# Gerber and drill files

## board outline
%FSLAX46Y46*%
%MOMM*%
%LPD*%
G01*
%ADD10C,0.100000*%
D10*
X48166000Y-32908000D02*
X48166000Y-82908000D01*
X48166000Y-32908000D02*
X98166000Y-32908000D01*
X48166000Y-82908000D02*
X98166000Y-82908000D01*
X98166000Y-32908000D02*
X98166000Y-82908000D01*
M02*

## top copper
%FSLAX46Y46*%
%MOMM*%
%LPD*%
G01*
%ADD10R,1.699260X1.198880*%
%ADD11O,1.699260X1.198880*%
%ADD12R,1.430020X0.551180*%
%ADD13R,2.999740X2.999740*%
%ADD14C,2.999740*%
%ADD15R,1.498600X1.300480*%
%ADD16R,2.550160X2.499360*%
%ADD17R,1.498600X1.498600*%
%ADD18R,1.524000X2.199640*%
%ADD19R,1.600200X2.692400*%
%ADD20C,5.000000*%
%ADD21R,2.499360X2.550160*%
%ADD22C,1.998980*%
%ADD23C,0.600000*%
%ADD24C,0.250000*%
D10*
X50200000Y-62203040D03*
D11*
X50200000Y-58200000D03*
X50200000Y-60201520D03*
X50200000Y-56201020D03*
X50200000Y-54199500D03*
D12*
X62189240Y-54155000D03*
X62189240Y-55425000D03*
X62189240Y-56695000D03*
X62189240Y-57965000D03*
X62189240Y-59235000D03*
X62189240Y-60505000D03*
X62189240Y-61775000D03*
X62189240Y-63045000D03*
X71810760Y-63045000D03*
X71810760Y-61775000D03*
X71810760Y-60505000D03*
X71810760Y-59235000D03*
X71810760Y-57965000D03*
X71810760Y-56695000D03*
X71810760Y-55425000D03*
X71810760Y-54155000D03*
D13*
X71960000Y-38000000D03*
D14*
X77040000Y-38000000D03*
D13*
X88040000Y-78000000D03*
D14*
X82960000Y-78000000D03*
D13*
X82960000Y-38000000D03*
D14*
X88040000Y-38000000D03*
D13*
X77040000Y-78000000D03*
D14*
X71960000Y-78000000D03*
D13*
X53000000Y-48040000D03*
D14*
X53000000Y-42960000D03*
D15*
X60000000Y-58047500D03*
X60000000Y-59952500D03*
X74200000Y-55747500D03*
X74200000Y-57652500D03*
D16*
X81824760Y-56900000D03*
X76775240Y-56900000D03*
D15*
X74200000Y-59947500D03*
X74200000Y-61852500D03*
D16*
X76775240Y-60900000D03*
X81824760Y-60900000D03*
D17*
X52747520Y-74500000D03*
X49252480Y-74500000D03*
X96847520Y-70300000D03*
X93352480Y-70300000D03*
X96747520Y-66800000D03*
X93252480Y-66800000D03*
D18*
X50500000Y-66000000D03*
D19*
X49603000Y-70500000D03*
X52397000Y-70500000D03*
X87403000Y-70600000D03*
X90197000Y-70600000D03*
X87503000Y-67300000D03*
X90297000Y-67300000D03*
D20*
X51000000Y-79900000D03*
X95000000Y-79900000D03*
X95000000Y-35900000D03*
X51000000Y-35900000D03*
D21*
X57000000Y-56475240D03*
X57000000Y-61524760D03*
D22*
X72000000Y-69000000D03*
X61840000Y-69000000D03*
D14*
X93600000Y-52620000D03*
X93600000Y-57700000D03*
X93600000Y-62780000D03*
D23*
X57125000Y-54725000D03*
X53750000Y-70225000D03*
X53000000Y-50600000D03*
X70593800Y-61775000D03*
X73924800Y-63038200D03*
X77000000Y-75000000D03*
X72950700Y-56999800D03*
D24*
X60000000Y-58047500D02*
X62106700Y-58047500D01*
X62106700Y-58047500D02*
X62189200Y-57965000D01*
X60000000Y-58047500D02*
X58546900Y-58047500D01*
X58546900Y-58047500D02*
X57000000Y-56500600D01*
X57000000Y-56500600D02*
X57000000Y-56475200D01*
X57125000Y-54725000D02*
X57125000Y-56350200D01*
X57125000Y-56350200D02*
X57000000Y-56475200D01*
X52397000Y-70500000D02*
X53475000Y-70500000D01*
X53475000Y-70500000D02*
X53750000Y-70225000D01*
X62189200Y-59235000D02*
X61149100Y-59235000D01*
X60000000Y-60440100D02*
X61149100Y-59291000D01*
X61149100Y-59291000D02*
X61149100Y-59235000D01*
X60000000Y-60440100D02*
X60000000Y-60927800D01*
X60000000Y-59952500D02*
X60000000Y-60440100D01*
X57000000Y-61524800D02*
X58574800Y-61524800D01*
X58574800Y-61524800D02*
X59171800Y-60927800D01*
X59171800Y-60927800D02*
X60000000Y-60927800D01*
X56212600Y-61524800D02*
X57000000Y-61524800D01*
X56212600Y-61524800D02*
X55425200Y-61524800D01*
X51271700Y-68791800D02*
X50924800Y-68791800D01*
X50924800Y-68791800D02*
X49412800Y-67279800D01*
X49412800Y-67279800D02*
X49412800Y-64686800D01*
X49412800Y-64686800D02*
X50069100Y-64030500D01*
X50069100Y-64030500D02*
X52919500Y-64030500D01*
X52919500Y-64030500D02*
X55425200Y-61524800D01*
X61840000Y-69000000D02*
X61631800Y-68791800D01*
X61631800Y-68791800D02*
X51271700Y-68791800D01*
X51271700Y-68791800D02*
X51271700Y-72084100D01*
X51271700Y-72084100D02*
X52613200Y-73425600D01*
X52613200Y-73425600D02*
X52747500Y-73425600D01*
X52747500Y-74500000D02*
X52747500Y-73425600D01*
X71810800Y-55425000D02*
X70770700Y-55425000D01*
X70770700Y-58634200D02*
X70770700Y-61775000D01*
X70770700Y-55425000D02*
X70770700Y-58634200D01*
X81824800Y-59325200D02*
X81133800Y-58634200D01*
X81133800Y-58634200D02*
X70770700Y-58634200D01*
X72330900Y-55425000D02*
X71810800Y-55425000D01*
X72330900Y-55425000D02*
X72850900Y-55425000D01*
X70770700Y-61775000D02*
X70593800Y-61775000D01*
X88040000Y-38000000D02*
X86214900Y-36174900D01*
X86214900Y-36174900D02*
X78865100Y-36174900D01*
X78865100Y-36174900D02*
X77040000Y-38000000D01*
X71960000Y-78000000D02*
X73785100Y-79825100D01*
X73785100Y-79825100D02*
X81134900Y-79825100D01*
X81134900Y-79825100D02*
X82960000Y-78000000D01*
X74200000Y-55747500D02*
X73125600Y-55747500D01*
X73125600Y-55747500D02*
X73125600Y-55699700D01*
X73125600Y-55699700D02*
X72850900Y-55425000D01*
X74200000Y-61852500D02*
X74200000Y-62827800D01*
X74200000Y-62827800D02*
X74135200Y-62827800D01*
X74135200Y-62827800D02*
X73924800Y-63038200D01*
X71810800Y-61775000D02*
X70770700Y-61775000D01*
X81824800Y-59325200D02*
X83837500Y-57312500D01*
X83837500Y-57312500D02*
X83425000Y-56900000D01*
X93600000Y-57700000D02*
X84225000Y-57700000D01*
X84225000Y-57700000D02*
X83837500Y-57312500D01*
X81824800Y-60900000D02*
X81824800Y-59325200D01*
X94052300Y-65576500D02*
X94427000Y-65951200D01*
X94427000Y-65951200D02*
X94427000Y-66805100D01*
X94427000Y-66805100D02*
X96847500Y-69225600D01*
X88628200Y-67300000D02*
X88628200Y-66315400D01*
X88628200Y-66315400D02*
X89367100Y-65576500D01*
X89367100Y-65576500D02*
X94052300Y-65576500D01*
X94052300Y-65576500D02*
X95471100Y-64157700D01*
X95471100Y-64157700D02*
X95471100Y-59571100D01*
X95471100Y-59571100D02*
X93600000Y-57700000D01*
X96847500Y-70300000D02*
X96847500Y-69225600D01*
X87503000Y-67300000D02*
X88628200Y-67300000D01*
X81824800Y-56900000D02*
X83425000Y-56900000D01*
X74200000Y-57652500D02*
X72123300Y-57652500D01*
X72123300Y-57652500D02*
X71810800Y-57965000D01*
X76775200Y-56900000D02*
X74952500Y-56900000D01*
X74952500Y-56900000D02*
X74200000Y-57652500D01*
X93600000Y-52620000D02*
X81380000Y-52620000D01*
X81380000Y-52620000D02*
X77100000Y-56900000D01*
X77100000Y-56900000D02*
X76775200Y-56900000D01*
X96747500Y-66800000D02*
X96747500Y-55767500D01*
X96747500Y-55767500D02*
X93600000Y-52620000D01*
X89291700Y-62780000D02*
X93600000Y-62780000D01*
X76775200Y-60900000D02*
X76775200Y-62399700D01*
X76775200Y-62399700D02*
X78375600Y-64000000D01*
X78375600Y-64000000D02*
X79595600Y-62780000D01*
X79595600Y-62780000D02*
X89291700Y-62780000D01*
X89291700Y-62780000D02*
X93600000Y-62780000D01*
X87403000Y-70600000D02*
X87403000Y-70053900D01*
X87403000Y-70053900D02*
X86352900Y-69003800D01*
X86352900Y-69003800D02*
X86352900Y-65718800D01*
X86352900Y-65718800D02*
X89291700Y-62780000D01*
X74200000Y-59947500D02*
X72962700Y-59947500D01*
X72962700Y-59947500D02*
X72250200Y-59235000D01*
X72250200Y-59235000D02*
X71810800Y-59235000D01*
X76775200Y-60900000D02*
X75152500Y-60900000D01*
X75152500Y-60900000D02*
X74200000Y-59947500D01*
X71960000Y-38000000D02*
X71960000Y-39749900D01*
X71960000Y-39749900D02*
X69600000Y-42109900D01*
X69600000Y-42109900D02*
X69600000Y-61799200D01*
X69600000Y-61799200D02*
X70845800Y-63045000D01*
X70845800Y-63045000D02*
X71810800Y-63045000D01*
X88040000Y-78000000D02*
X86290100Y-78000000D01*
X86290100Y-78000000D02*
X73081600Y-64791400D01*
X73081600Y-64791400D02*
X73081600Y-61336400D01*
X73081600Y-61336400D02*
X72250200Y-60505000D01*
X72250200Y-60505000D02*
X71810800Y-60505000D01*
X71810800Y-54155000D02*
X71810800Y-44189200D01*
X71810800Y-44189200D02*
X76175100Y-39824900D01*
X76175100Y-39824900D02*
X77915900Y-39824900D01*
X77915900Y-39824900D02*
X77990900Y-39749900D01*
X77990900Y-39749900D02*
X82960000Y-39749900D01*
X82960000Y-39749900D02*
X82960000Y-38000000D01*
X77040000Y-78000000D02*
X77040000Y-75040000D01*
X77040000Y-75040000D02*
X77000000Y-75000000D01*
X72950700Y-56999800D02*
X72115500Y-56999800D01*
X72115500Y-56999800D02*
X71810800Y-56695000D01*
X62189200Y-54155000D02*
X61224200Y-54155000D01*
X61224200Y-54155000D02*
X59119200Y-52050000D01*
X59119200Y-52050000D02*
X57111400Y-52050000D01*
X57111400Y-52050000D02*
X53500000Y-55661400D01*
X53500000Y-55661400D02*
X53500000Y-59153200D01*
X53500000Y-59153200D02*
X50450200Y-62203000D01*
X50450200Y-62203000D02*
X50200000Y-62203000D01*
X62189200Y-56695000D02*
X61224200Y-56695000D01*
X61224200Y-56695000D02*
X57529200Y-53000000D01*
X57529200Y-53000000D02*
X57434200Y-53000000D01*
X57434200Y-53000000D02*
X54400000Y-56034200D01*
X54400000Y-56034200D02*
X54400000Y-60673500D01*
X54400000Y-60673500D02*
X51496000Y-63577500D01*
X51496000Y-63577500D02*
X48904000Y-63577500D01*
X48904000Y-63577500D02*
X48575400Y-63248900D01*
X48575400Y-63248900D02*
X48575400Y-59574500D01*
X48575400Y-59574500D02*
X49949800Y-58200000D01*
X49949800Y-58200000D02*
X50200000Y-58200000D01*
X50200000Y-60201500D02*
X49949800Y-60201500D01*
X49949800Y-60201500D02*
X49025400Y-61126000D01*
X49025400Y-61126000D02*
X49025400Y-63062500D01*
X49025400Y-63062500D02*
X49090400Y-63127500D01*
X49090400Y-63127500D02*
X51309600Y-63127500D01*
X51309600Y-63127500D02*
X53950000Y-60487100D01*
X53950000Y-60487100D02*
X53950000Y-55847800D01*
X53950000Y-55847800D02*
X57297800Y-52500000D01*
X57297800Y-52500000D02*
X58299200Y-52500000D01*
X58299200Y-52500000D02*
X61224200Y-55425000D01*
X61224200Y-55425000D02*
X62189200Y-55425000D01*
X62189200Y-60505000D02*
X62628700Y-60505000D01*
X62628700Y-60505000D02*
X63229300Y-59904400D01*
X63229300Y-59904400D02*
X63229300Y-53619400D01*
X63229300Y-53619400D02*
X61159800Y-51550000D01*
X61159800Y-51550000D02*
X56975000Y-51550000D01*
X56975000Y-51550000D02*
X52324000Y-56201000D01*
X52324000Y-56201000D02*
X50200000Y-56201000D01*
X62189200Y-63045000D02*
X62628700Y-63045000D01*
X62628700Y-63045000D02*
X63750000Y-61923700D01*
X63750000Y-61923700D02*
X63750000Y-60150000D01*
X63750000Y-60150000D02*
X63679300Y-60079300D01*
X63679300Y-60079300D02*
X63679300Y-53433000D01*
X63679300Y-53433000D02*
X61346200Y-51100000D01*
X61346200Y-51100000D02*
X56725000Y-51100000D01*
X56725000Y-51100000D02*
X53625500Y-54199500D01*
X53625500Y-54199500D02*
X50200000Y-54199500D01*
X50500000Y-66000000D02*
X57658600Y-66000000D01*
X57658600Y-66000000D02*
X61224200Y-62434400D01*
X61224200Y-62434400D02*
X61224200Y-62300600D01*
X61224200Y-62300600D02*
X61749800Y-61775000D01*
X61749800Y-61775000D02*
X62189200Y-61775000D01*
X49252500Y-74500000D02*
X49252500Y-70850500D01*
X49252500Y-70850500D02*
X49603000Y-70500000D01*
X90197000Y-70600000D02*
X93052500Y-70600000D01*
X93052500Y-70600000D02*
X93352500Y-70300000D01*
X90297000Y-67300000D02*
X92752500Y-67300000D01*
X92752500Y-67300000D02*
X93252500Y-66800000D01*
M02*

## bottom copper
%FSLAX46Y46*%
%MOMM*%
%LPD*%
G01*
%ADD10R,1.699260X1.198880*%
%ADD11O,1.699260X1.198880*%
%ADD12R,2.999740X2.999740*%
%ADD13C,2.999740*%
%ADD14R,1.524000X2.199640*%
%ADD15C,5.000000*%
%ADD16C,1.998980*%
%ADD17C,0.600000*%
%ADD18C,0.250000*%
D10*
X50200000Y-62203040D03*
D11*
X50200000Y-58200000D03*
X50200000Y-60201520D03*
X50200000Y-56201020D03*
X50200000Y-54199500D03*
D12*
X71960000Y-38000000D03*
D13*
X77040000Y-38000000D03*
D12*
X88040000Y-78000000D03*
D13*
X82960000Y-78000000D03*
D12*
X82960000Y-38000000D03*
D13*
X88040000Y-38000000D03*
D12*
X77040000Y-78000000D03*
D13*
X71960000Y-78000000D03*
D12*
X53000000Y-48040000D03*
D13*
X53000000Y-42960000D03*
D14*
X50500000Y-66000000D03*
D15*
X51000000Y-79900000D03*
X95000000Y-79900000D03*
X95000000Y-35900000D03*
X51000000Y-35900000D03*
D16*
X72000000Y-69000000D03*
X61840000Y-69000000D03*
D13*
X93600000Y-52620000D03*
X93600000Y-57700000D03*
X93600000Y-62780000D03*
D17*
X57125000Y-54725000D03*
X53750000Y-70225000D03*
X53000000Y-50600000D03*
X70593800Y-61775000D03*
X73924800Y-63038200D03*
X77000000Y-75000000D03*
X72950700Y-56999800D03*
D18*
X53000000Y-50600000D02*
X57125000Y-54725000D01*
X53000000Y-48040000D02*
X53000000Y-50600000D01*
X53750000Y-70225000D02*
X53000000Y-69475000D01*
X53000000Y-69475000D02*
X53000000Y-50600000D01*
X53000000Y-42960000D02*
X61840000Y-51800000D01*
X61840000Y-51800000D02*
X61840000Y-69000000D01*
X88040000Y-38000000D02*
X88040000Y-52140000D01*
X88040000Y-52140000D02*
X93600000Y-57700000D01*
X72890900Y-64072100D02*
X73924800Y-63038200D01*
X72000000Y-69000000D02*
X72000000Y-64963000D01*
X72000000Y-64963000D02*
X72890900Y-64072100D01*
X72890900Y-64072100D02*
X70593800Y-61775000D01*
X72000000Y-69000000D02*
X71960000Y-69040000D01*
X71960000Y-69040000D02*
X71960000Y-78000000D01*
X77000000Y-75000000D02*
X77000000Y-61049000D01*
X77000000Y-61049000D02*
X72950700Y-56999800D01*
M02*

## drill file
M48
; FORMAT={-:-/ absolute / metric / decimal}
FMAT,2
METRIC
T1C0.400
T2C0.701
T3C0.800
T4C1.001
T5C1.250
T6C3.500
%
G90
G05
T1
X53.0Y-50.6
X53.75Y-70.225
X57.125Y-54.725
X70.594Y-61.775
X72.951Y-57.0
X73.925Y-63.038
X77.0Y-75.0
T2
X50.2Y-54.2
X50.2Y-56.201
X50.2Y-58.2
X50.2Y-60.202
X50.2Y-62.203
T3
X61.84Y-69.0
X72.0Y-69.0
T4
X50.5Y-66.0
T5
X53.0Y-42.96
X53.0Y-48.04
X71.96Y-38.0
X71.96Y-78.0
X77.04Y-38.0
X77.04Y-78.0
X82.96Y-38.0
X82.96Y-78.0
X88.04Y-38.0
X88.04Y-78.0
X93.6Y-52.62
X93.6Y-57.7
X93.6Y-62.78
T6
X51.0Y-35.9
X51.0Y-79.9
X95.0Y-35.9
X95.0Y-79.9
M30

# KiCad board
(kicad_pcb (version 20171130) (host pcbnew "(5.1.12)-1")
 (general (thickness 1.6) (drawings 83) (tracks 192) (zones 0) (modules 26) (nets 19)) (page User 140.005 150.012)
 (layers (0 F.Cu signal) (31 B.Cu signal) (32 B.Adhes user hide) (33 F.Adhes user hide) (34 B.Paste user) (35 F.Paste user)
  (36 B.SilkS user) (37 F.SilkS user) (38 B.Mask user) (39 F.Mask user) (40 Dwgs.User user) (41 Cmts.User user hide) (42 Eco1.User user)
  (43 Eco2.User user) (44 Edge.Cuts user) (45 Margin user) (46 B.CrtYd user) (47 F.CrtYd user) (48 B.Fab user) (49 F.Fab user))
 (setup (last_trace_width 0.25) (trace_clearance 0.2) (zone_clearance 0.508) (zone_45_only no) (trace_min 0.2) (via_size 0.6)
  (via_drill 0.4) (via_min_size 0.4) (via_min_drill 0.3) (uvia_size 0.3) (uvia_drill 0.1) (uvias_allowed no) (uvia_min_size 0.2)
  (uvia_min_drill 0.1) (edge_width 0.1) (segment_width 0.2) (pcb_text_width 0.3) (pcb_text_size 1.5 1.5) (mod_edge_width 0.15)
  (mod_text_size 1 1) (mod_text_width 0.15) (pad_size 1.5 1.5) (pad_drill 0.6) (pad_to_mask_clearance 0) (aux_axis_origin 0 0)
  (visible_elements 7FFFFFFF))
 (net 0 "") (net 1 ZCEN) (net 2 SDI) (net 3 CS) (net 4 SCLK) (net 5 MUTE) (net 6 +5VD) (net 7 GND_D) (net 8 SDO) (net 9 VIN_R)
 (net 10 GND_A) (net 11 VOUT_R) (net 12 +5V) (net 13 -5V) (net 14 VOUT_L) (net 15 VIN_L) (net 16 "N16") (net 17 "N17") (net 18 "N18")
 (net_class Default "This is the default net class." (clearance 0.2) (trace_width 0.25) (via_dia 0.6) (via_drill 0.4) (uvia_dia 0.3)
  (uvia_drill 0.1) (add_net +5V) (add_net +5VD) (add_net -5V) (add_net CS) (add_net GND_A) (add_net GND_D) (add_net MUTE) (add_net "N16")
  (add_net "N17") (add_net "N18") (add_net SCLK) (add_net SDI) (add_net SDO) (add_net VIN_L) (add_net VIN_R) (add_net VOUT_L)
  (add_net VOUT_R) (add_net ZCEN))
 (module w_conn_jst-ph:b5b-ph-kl (layer F.Cu) (at 50.2 58.2 90)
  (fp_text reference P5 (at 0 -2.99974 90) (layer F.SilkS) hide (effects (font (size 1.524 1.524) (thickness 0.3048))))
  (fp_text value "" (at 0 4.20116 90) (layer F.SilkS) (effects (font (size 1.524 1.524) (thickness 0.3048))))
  (pad 1 thru_hole rect (at -4.00304 0 90) (size 1.19888 1.69926) (drill 0.70104) (layers *.Cu *.Mask F.SilkS) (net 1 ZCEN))
  (pad 3 thru_hole oval (at 0 0 90) (size 1.19888 1.69926) (drill 0.70104) (layers *.Cu *.Mask F.SilkS) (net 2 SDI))
  (pad 2 thru_hole oval (at -2.00152 0 90) (size 1.19888 1.69926) (drill 0.70104) (layers *.Cu *.Mask F.SilkS) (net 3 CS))
  (pad 4 thru_hole oval (at 1.99898 0 90) (size 1.19888 1.69926) (drill 0.70104) (layers *.Cu *.Mask F.SilkS) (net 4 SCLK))
  (pad 5 thru_hole oval (at 4.0005 0 90) (size 1.19888 1.69926) (drill 0.70104) (layers *.Cu *.Mask F.SilkS) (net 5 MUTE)))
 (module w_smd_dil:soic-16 (layer F.Cu) (at 67 58.6 270)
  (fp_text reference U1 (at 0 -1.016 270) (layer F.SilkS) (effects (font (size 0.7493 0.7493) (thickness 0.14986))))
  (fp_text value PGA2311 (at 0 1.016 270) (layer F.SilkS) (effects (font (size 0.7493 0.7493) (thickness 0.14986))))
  (pad 1 smd rect (at -4.445 4.81076 270) (size 0.55118 1.43002) (layers F.Cu F.Paste F.Mask) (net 1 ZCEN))
  (pad 2 smd rect (at -3.175 4.81076 270) (size 0.55118 1.43002) (layers F.Cu F.Paste F.Mask) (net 3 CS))
  (pad 3 smd rect (at -1.905 4.81076 270) (size 0.55118 1.43002) (layers F.Cu F.Paste F.Mask) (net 2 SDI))
  (pad 4 smd rect (at -0.635 4.81076 270) (size 0.55118 1.43002) (layers F.Cu F.Paste F.Mask) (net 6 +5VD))
  (pad 5 smd rect (at 0.635 4.81076 270) (size 0.55118 1.43002) (layers F.Cu F.Paste F.Mask) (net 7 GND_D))
  (pad 6 smd rect (at 1.905 4.81076 270) (size 0.55118 1.43002) (layers F.Cu F.Paste F.Mask) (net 4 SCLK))
  (pad 7 smd rect (at 3.175 4.81076 270) (size 0.55118 1.43002) (layers F.Cu F.Paste F.Mask) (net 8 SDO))
  (pad 8 smd rect (at 4.445 4.81076 270) (size 0.55118 1.43002) (layers F.Cu F.Paste F.Mask) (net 5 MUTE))
  (pad 9 smd rect (at 4.445 -4.81076 270) (size 0.55118 1.43002) (layers F.Cu F.Paste F.Mask) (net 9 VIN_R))
  (pad 10 smd rect (at 3.175 -4.81076 270) (size 0.55118 1.43002) (layers F.Cu F.Paste F.Mask) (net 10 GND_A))
  (pad 11 smd rect (at 1.905 -4.81076 270) (size 0.55118 1.43002) (layers F.Cu F.Paste F.Mask) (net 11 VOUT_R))
  (pad 12 smd rect (at 0.635 -4.81076 270) (size 0.55118 1.43002) (layers F.Cu F.Paste F.Mask) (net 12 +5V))
  (pad 13 smd rect (at -0.635 -4.81076 270) (size 0.55118 1.43002) (layers F.Cu F.Paste F.Mask) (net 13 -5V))
  (pad 14 smd rect (at -1.905 -4.81076 270) (size 0.55118 1.43002) (layers F.Cu F.Paste F.Mask) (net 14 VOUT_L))
  (pad 15 smd rect (at -3.175 -4.81076 270) (size 0.55118 1.43002) (layers F.Cu F.Paste F.Mask) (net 10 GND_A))
  (pad 16 smd rect (at -4.445 -4.81076 270) (size 0.55118 1.43002) (layers F.Cu F.Paste F.Mask) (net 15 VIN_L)))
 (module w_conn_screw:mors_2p (layer F.Cu) (at 74.5 38)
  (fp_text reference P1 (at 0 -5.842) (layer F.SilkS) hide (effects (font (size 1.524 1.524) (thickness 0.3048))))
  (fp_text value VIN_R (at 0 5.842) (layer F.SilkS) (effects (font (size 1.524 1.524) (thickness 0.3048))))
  (pad 1 thru_hole rect (at -2.54 0) (size 2.99974 2.99974) (drill 1.24968) (layers *.Cu *.Mask F.SilkS) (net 9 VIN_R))
  (pad 2 thru_hole circle (at 2.54 0) (size 2.99974 2.99974) (drill 1.24968) (layers *.Cu *.Mask F.SilkS) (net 10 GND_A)))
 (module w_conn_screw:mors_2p (layer F.Cu) (at 85.5 78 180)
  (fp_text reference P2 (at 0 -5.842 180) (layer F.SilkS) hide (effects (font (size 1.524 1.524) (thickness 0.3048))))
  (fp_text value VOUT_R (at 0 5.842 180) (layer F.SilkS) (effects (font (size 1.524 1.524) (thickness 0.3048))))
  (pad 1 thru_hole rect (at -2.54 0 180) (size 2.99974 2.99974) (drill 1.24968) (layers *.Cu *.Mask F.SilkS) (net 11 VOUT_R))
  (pad 2 thru_hole circle (at 2.54 0 180) (size 2.99974 2.99974) (drill 1.24968) (layers *.Cu *.Mask F.SilkS) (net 10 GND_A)))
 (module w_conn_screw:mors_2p (layer F.Cu) (at 85.5 38)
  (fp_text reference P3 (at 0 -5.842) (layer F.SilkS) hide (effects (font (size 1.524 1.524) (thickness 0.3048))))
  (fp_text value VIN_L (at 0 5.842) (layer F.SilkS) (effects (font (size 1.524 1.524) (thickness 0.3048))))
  (pad 1 thru_hole rect (at -2.54 0) (size 2.99974 2.99974) (drill 1.24968) (layers *.Cu *.Mask F.SilkS) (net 15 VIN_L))
  (pad 2 thru_hole circle (at 2.54 0) (size 2.99974 2.99974) (drill 1.24968) (layers *.Cu *.Mask F.SilkS) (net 10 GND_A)))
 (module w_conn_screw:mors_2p (layer F.Cu) (at 74.5 78 180)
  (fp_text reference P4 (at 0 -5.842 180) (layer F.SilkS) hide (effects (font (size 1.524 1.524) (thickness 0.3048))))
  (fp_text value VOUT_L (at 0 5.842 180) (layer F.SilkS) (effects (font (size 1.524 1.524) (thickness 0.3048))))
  (pad 1 thru_hole rect (at -2.54 0 180) (size 2.99974 2.99974) (drill 1.24968) (layers *.Cu *.Mask F.SilkS) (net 14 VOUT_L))
  (pad 2 thru_hole circle (at 2.54 0 180) (size 2.99974 2.99974) (drill 1.24968) (layers *.Cu *.Mask F.SilkS) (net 10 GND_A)))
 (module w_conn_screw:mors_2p (layer F.Cu) (at 53 45.5 90)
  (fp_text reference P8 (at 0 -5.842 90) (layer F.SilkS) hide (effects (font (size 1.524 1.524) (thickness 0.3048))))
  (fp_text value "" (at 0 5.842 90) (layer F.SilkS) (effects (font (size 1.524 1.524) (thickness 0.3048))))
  (pad 1 thru_hole rect (at -2.54 0 90) (size 2.99974 2.99974) (drill 1.24968) (layers *.Cu *.Mask F.SilkS) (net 6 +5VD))
  (pad 2 thru_hole circle (at 2.54 0 90) (size 2.99974 2.99974) (drill 1.24968) (layers *.Cu *.Mask F.SilkS) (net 7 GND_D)))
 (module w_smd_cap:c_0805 (layer F.Cu) (at 60 59 90)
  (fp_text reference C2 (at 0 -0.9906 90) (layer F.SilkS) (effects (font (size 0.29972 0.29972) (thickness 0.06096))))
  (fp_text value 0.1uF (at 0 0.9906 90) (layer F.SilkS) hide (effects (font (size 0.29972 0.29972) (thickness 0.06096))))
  (pad 1 smd rect (at 0.9525 0 90) (size 1.30048 1.4986) (layers F.Cu F.Paste F.Mask) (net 6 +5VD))
  (pad 2 smd rect (at -0.9525 0 90) (size 1.30048 1.4986) (layers F.Cu F.Paste F.Mask) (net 7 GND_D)))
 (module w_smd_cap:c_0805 (layer F.Cu) (at 74.2 56.7 90)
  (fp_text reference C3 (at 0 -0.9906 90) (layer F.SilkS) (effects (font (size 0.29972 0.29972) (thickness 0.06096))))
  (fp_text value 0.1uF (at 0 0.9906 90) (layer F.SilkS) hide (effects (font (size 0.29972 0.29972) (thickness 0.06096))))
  (pad 1 smd rect (at 0.9525 0 90) (size 1.30048 1.4986) (layers F.Cu F.Paste F.Mask) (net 10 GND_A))
  (pad 2 smd rect (at -0.9525 0 90) (size 1.30048 1.4986) (layers F.Cu F.Paste F.Mask) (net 13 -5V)))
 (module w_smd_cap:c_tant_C (layer F.Cu) (at 79.3 56.9)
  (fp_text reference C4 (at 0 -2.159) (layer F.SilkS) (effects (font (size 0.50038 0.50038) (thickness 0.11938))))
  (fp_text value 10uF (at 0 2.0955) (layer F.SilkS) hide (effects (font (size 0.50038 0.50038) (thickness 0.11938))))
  (pad 1 smd rect (at 2.52476 0) (size 2.55016 2.49936) (layers F.Cu F.Paste F.Mask) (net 10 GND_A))
  (pad 2 smd rect (at -2.52476 0) (size 2.55016 2.49936) (layers F.Cu F.Paste F.Mask) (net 13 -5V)))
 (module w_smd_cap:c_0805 (layer F.Cu) (at 74.2 60.9 90)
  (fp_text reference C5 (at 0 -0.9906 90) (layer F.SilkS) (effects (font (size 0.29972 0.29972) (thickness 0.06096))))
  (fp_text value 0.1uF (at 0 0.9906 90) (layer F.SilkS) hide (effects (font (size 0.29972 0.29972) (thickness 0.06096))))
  (pad 1 smd rect (at 0.9525 0 90) (size 1.30048 1.4986) (layers F.Cu F.Paste F.Mask) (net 12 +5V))
  (pad 2 smd rect (at -0.9525 0 90) (size 1.30048 1.4986) (layers F.Cu F.Paste F.Mask) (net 10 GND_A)))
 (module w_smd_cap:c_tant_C (layer F.Cu) (at 79.3 60.9 180)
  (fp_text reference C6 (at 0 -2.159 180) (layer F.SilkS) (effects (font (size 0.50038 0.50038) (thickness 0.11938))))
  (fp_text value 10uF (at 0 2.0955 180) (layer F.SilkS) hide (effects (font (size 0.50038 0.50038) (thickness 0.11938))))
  (pad 1 smd rect (at 2.52476 0 180) (size 2.55016 2.49936) (layers F.Cu F.Paste F.Mask) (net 12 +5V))
  (pad 2 smd rect (at -2.52476 0 180) (size 2.55016 2.49936) (layers F.Cu F.Paste F.Mask) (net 10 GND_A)))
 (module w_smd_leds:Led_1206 (layer F.Cu) (at 51 74.5 180)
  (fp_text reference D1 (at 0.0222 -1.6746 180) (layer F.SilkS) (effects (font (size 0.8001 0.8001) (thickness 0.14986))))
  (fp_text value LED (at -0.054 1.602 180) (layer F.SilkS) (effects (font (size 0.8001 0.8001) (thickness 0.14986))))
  (pad 1 smd rect (at -1.74752 0 180) (size 1.4986 1.4986) (layers F.Cu F.Paste F.Mask) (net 7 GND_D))
  (pad 2 smd rect (at 1.74752 0 180) (size 1.4986 1.4986) (layers F.Cu F.Paste F.Mask) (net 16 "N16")))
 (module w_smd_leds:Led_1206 (layer F.Cu) (at 95.1 70.3 180)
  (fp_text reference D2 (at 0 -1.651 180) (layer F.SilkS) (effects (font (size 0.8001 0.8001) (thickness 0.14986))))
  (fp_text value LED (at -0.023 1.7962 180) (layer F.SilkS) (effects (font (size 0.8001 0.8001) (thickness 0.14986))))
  (pad 1 smd rect (at -1.74752 0 180) (size 1.4986 1.4986) (layers F.Cu F.Paste F.Mask) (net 10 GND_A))
  (pad 2 smd rect (at 1.74752 0 180) (size 1.4986 1.4986) (layers F.Cu F.Paste F.Mask) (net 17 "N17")))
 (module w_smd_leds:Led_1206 (layer F.Cu) (at 95 66.8 180)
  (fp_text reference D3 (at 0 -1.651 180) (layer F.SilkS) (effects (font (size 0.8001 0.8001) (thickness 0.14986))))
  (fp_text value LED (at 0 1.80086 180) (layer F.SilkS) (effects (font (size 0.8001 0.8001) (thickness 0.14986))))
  (pad 1 smd rect (at -1.74752 0 180) (size 1.4986 1.4986) (layers F.Cu F.Paste F.Mask) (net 13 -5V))
  (pad 2 smd rect (at 1.74752 0 180) (size 1.4986 1.4986) (layers F.Cu F.Paste F.Mask) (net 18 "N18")))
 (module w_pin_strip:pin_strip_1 (layer F.Cu) (at 50.5 66)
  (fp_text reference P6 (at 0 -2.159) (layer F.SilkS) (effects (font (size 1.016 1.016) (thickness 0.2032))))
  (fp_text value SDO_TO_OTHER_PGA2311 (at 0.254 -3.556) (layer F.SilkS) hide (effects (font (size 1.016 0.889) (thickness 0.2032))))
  (pad 1 thru_hole rect (at 0 0) (size 1.524 2.19964) (drill 1.00076) (layers *.Cu *.Mask F.SilkS) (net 8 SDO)))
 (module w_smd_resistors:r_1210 (layer F.Cu) (at 51 70.5 180)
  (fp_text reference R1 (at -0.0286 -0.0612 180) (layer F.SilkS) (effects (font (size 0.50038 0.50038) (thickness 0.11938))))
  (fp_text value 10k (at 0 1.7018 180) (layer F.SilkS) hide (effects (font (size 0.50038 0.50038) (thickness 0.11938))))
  (pad 1 smd rect (at 1.397 0 180) (size 1.6002 2.6924) (layers F.Cu F.Paste F.Mask) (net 16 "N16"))
  (pad 2 smd rect (at -1.397 0 180) (size 1.6002 2.6924) (layers F.Cu F.Paste F.Mask) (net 6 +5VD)))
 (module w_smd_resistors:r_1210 (layer F.Cu) (at 88.8 70.6 180)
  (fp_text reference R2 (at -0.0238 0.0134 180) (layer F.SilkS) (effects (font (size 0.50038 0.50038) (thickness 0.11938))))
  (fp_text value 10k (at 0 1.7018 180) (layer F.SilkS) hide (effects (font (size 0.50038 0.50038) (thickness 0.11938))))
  (pad 1 smd rect (at 1.397 0 180) (size 1.6002 2.6924) (layers F.Cu F.Paste F.Mask) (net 12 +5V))
  (pad 2 smd rect (at -1.397 0 180) (size 1.6002 2.6924) (layers F.Cu F.Paste F.Mask) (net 17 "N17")))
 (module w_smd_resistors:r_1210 (layer F.Cu) (at 88.9 67.3 180)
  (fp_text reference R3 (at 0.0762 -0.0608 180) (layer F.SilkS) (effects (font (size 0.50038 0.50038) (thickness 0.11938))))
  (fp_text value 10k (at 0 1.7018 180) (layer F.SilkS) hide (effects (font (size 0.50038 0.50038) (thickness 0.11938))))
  (pad 1 smd rect (at 1.397 0 180) (size 1.6002 2.6924) (layers F.Cu F.Paste F.Mask) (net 10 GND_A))
  (pad 2 smd rect (at -1.397 0 180) (size 1.6002 2.6924) (layers F.Cu F.Paste F.Mask) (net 18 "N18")))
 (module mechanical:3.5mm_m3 (layer F.Cu) (at 51 80)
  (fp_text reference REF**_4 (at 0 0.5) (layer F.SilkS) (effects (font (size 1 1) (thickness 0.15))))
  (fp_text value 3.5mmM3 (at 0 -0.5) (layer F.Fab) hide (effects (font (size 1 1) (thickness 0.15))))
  (pad 1 thru_hole circle (at 0 -0.1) (size 5 5) (drill 3.5) (layers *.Cu *.Mask F.SilkS)))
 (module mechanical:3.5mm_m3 (layer F.Cu) (at 95 80)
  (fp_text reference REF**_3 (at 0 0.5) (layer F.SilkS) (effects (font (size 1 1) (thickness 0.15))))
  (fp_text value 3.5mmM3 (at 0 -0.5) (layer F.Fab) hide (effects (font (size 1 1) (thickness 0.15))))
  (pad 1 thru_hole circle (at 0 -0.1) (size 5 5) (drill 3.5) (layers *.Cu *.Mask F.SilkS)))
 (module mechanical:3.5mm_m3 (layer F.Cu) (at 95 36)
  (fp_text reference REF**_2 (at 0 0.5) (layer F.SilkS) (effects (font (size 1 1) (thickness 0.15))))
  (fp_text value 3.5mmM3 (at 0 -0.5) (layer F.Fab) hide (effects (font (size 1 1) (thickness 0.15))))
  (pad 1 thru_hole circle (at 0 -0.1) (size 5 5) (drill 3.5) (layers *.Cu *.Mask F.SilkS)))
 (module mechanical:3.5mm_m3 (layer F.Cu) (at 51 36)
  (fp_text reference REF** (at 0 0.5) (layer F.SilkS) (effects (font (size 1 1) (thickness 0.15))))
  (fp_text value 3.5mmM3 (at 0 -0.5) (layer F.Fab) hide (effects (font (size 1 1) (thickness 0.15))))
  (pad 1 thru_hole circle (at 0 -0.1) (size 5 5) (drill 3.5) (layers *.Cu *.Mask F.SilkS)))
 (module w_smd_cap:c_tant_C (layer F.Cu) (at 57 59 90)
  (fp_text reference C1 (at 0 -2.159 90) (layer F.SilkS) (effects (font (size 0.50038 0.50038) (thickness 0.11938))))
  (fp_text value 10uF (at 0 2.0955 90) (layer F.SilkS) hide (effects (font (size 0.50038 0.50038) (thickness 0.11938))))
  (pad 1 smd rect (at 2.52476 0 90) (size 2.55016 2.49936) (layers F.Cu F.Paste F.Mask) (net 6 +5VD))
  (pad 2 smd rect (at -2.52476 0 90) (size 2.55016 2.49936) (layers F.Cu F.Paste F.Mask) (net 7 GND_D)))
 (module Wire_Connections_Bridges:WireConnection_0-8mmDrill (layer F.Cu) (at 72 69 180)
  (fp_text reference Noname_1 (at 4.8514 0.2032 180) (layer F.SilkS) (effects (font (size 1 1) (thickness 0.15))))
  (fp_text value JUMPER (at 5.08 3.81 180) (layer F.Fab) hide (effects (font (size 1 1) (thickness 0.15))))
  (pad 1 thru_hole circle (at 0 0 180) (size 1.99898 1.99898) (drill 0.8001) (layers *.Cu *.Mask F.SilkS) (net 10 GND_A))
  (pad 2 thru_hole circle (at 10.16 0 180) (size 1.99898 1.99898) (drill 0.8001) (layers *.Cu *.Mask F.SilkS) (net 7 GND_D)))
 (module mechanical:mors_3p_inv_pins (layer F.Cu) (at 93.6 57.7 270)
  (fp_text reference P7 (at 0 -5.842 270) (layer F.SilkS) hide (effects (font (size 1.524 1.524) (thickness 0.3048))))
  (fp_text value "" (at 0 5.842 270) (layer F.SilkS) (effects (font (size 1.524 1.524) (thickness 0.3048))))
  (pad 3 thru_hole circle (at -5.08 0 270) (size 2.99974 2.99974) (drill 1.24968) (layers *.Cu *.Mask F.SilkS) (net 13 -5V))
  (pad 2 thru_hole circle (at 0 0 270) (size 2.99974 2.99974) (drill 1.24968) (layers *.Cu *.Mask F.SilkS) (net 10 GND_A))
  (pad 1 thru_hole circle (at 5.08 0 270) (size 2.99974 2.99974) (drill 1.24968) (layers *.Cu *.Mask F.SilkS) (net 12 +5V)))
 (gr_line (start 48.166 32.908) (end 48.166 82.908) (angle 90) (layer Edge.Cuts) (width 0.1))
 (gr_line (start 48.166 32.908) (end 98.166 32.908) (angle 90) (layer Edge.Cuts) (width 0.1))
 (gr_line (start 48.166 82.908) (end 98.166 82.908) (angle 90) (layer Edge.Cuts) (width 0.1))
 (gr_line (start 98.166 32.908) (end 98.166 82.908) (angle 90) (layer Edge.Cuts) (width 0.1))
 (segment (start 53 50.6) (end 57.125 54.725) (width 0.25) (layer B.Cu) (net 6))
 (segment (start 53 48.04) (end 53 50.6) (width 0.25) (layer B.Cu) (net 6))
 (segment (start 60 58.0475) (end 62.1067 58.0475) (width 0.25) (layer F.Cu) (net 6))
 (segment (start 62.1067 58.0475) (end 62.1892 57.965) (width 0.25) (layer F.Cu) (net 6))
 (segment (start 60 58.0475) (end 58.5469 58.0475) (width 0.25) (layer F.Cu) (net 6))
 (segment (start 58.5469 58.0475) (end 57 56.5006) (width 0.25) (layer F.Cu) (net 6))
 (segment (start 57 56.5006) (end 57 56.4752) (width 0.25) (layer F.Cu) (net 6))
 (segment (start 57.125 54.725) (end 57.125 56.3502) (width 0.25) (layer F.Cu) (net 6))
 (segment (start 57.125 56.3502) (end 57 56.4752) (width 0.25) (layer F.Cu) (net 6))
 (segment (start 52.397 70.5) (end 53.475 70.5) (width 0.25) (layer F.Cu) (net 6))
 (segment (start 53.475 70.5) (end 53.75 70.225) (width 0.25) (layer F.Cu) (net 6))
 (segment (start 53.75 70.225) (end 53 69.475) (width 0.25) (layer B.Cu) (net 6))
 (segment (start 53 69.475) (end 53 50.6) (width 0.25) (layer B.Cu) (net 6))
 (via (at 57.125 54.725) (size 0.6) (layers F.Cu B.Cu) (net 6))
 (via (at 53.75 70.225) (size 0.6) (layers F.Cu B.Cu) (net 6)) (via (at 53 50.6) (size 0.6) (layers F.Cu B.Cu) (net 6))
 (segment (start 53 42.96) (end 61.84 51.8) (width 0.25) (layer B.Cu) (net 7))
 (segment (start 61.84 51.8) (end 61.84 69) (width 0.25) (layer B.Cu) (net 7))
 (segment (start 62.1892 59.235) (end 61.1491 59.235) (width 0.25) (layer F.Cu) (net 7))
 (segment (start 60 60.4401) (end 61.1491 59.291) (width 0.25) (layer F.Cu) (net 7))
 (segment (start 61.1491 59.291) (end 61.1491 59.235) (width 0.25) (layer F.Cu) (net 7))
 (segment (start 60 60.4401) (end 60 60.9278) (width 0.25) (layer F.Cu) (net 7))
 (segment (start 60 59.9525) (end 60 60.4401) (width 0.25) (layer F.Cu) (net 7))
 (segment (start 57 61.5248) (end 58.5748 61.5248) (width 0.25) (layer F.Cu) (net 7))
 (segment (start 58.5748 61.5248) (end 59.1718 60.9278) (width 0.25) (layer F.Cu) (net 7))
 (segment (start 59.1718 60.9278) (end 60 60.9278) (width 0.25) (layer F.Cu) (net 7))
 (segment (start 56.2126 61.5248) (end 57 61.5248) (width 0.25) (layer F.Cu) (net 7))
 (segment (start 56.2126 61.5248) (end 55.4252 61.5248) (width 0.25) (layer F.Cu) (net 7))
 (segment (start 51.2717 68.7918) (end 50.9248 68.7918) (width 0.25) (layer F.Cu) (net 7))
 (segment (start 50.9248 68.7918) (end 49.4128 67.2798) (width 0.25) (layer F.Cu) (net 7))
 (segment (start 49.4128 67.2798) (end 49.4128 64.6868) (width 0.25) (layer F.Cu) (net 7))
 (segment (start 49.4128 64.6868) (end 50.0691 64.0305) (width 0.25) (layer F.Cu) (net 7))
 (segment (start 50.0691 64.0305) (end 52.9195 64.0305) (width 0.25) (layer F.Cu) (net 7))
 (segment (start 52.9195 64.0305) (end 55.4252 61.5248) (width 0.25) (layer F.Cu) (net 7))
 (segment (start 61.84 69) (end 61.6318 68.7918) (width 0.25) (layer F.Cu) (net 7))
 (segment (start 61.6318 68.7918) (end 51.2717 68.7918) (width 0.25) (layer F.Cu) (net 7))
 (segment (start 51.2717 68.7918) (end 51.2717 72.0841) (width 0.25) (layer F.Cu) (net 7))
 (segment (start 51.2717 72.0841) (end 52.6132 73.4256) (width 0.25) (layer F.Cu) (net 7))
 (segment (start 52.6132 73.4256) (end 52.7475 73.4256) (width 0.25) (layer F.Cu) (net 7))
 (segment (start 52.7475 74.5) (end 52.7475 73.4256) (width 0.25) (layer F.Cu) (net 7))
 (segment (start 71.8108 55.425) (end 70.7707 55.425) (width 0.25) (layer F.Cu) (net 10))
 (segment (start 70.7707 58.6342) (end 70.7707 61.775) (width 0.25) (layer F.Cu) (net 10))
 (segment (start 70.7707 55.425) (end 70.7707 58.6342) (width 0.25) (layer F.Cu) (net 10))
 (segment (start 81.8248 59.3252) (end 81.1338 58.6342) (width 0.25) (layer F.Cu) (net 10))
 (segment (start 81.1338 58.6342) (end 70.7707 58.6342) (width 0.25) (layer F.Cu) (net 10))
 (segment (start 72.3309 55.425) (end 71.8108 55.425) (width 0.25) (layer F.Cu) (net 10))
 (segment (start 72.3309 55.425) (end 72.8509 55.425) (width 0.25) (layer F.Cu) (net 10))
 (segment (start 88.04 38) (end 88.04 52.14) (width 0.25) (layer B.Cu) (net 10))
 (segment (start 88.04 52.14) (end 93.6 57.7) (width 0.25) (layer B.Cu) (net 10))
 (segment (start 72.8909 64.0721) (end 73.9248 63.0382) (width 0.25) (layer B.Cu) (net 10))
 (segment (start 72 69) (end 72 64.963) (width 0.25) (layer B.Cu) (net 10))
 (segment (start 72 64.963) (end 72.8909 64.0721) (width 0.25) (layer B.Cu) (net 10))
 (segment (start 72.8909 64.0721) (end 70.5938 61.775) (width 0.25) (layer B.Cu) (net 10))
 (segment (start 70.7707 61.775) (end 70.5938 61.775) (width 0.25) (layer F.Cu) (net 10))
 (segment (start 88.04 38) (end 86.2149 36.1749) (width 0.25) (layer F.Cu) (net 10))
 (segment (start 86.2149 36.1749) (end 78.8651 36.1749) (width 0.25) (layer F.Cu) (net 10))
 (segment (start 78.8651 36.1749) (end 77.04 38) (width 0.25) (layer F.Cu) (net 10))
 (segment (start 71.96 78) (end 73.7851 79.8251) (width 0.25) (layer F.Cu) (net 10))
 (segment (start 73.7851 79.8251) (end 81.1349 79.8251) (width 0.25) (layer F.Cu) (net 10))
 (segment (start 81.1349 79.8251) (end 82.96 78) (width 0.25) (layer F.Cu) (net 10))
 (segment (start 74.2 55.7475) (end 73.1256 55.7475) (width 0.25) (layer F.Cu) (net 10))
 (segment (start 73.1256 55.7475) (end 73.1256 55.6997) (width 0.25) (layer F.Cu) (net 10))
 (segment (start 73.1256 55.6997) (end 72.8509 55.425) (width 0.25) (layer F.Cu) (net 10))
 (segment (start 74.2 61.8525) (end 74.2 62.8278) (width 0.25) (layer F.Cu) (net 10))
 (segment (start 74.2 62.8278) (end 74.1352 62.8278) (width 0.25) (layer F.Cu) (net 10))
 (segment (start 74.1352 62.8278) (end 73.9248 63.0382) (width 0.25) (layer F.Cu) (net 10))
 (segment (start 71.8108 61.775) (end 70.7707 61.775) (width 0.25) (layer F.Cu) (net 10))
 (segment (start 81.8248 59.3252) (end 83.8375 57.3125) (width 0.25) (layer F.Cu) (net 10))
 (segment (start 83.8375 57.3125) (end 83.425 56.9) (width 0.25) (layer F.Cu) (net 10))
 (segment (start 93.6 57.7) (end 84.225 57.7) (width 0.25) (layer F.Cu) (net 10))
 (segment (start 84.225 57.7) (end 83.8375 57.3125) (width 0.25) (layer F.Cu) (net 10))
 (segment (start 81.8248 60.9) (end 81.8248 59.3252) (width 0.25) (layer F.Cu) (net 10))
 (segment (start 94.0523 65.5765) (end 94.427 65.9512) (width 0.25) (layer F.Cu) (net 10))
 (segment (start 94.427 65.9512) (end 94.427 66.8051) (width 0.25) (layer F.Cu) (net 10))
 (segment (start 94.427 66.8051) (end 96.8475 69.2256) (width 0.25) (layer F.Cu) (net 10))
 (segment (start 88.6282 67.3) (end 88.6282 66.3154) (width 0.25) (layer F.Cu) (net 10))
 (segment (start 88.6282 66.3154) (end 89.3671 65.5765) (width 0.25) (layer F.Cu) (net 10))
 (segment (start 89.3671 65.5765) (end 94.0523 65.5765) (width 0.25) (layer F.Cu) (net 10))
 (segment (start 94.0523 65.5765) (end 95.4711 64.1577) (width 0.25) (layer F.Cu) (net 10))
 (segment (start 95.4711 64.1577) (end 95.4711 59.5711) (width 0.25) (layer F.Cu) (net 10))
 (segment (start 95.4711 59.5711) (end 93.6 57.7) (width 0.25) (layer F.Cu) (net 10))
 (segment (start 96.8475 70.3) (end 96.8475 69.2256) (width 0.25) (layer F.Cu) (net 10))
 (segment (start 87.503 67.3) (end 88.6282 67.3) (width 0.25) (layer F.Cu) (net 10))
 (segment (start 72 69) (end 71.96 69.04) (width 0.25) (layer B.Cu) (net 10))
 (segment (start 71.96 69.04) (end 71.96 78) (width 0.25) (layer B.Cu) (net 10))
 (segment (start 81.8248 56.9) (end 83.425 56.9) (width 0.25) (layer F.Cu) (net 10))
 (via (at 70.5938 61.775) (size 0.6) (layers F.Cu B.Cu) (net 10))
 (via (at 73.9248 63.0382) (size 0.6) (layers F.Cu B.Cu) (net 10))
 (segment (start 74.2 57.6525) (end 72.1233 57.6525) (width 0.25) (layer F.Cu) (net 13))
 (segment (start 72.1233 57.6525) (end 71.8108 57.965) (width 0.25) (layer F.Cu) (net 13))
 (segment (start 76.7752 56.9) (end 74.9525 56.9) (width 0.25) (layer F.Cu) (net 13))
 (segment (start 74.9525 56.9) (end 74.2 57.6525) (width 0.25) (layer F.Cu) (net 13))
 (segment (start 93.6 52.62) (end 81.38 52.62) (width 0.25) (layer F.Cu) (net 13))
 (segment (start 81.38 52.62) (end 77.1 56.9) (width 0.25) (layer F.Cu) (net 13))
 (segment (start 77.1 56.9) (end 76.7752 56.9) (width 0.25) (layer F.Cu) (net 13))
 (segment (start 96.7475 66.8) (end 96.7475 55.7675) (width 0.25) (layer F.Cu) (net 13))
 (segment (start 96.7475 55.7675) (end 93.6 52.62) (width 0.25) (layer F.Cu) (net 13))
 (segment (start 89.2917 62.78) (end 93.6 62.78) (width 0.25) (layer F.Cu) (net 12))
 (segment (start 76.7752 60.9) (end 76.7752 62.3997) (width 0.25) (layer F.Cu) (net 12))
 (segment (start 76.7752 62.3997) (end 78.3756 64) (width 0.25) (layer F.Cu) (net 12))
 (segment (start 78.3756 64) (end 79.5956 62.78) (width 0.25) (layer F.Cu) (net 12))
 (segment (start 79.5956 62.78) (end 89.2917 62.78) (width 0.25) (layer F.Cu) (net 12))
 (segment (start 89.2917 62.78) (end 93.6 62.78) (width 0.25) (layer F.Cu) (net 12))
 (segment (start 87.403 70.6) (end 87.403 70.0539) (width 0.25) (layer F.Cu) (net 12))
 (segment (start 87.403 70.0539) (end 86.3529 69.0038) (width 0.25) (layer F.Cu) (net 12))
 (segment (start 86.3529 69.0038) (end 86.3529 65.7188) (width 0.25) (layer F.Cu) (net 12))
 (segment (start 86.3529 65.7188) (end 89.2917 62.78) (width 0.25) (layer F.Cu) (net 12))
 (segment (start 74.2 59.9475) (end 72.9627 59.9475) (width 0.25) (layer F.Cu) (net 12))
 (segment (start 72.9627 59.9475) (end 72.2502 59.235) (width 0.25) (layer F.Cu) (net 12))
 (segment (start 72.2502 59.235) (end 71.8108 59.235) (width 0.25) (layer F.Cu) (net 12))
 (segment (start 76.7752 60.9) (end 75.1525 60.9) (width 0.25) (layer F.Cu) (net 12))
 (segment (start 75.1525 60.9) (end 74.2 59.9475) (width 0.25) (layer F.Cu) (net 12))
 (segment (start 71.96 38) (end 71.96 39.7499) (width 0.25) (layer F.Cu) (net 9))
 (segment (start 71.96 39.7499) (end 69.6 42.1099) (width 0.25) (layer F.Cu) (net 9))
 (segment (start 69.6 42.1099) (end 69.6 61.7992) (width 0.25) (layer F.Cu) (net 9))
 (segment (start 69.6 61.7992) (end 70.8458 63.045) (width 0.25) (layer F.Cu) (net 9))
 (segment (start 70.8458 63.045) (end 71.8108 63.045) (width 0.25) (layer F.Cu) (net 9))
 (segment (start 88.04 78) (end 86.2901 78) (width 0.25) (layer F.Cu) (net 11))
 (segment (start 86.2901 78) (end 73.0816 64.7914) (width 0.25) (layer F.Cu) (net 11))
 (segment (start 73.0816 64.7914) (end 73.0816 61.3364) (width 0.25) (layer F.Cu) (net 11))
 (segment (start 73.0816 61.3364) (end 72.2502 60.505) (width 0.25) (layer F.Cu) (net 11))
 (segment (start 72.2502 60.505) (end 71.8108 60.505) (width 0.25) (layer F.Cu) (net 11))
 (segment (start 71.8108 54.155) (end 71.8108 44.1892) (width 0.25) (layer F.Cu) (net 15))
 (segment (start 71.8108 44.1892) (end 76.1751 39.8249) (width 0.25) (layer F.Cu) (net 15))
 (segment (start 76.1751 39.8249) (end 77.9159 39.8249) (width 0.25) (layer F.Cu) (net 15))
 (segment (start 77.9159 39.8249) (end 77.9909 39.7499) (width 0.25) (layer F.Cu) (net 15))
 (segment (start 77.9909 39.7499) (end 82.96 39.7499) (width 0.25) (layer F.Cu) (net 15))
 (segment (start 82.96 39.7499) (end 82.96 38) (width 0.25) (layer F.Cu) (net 15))
 (segment (start 77.04 78) (end 77.04 75.04) (width 0.25) (layer F.Cu) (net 14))
 (segment (start 77.04 75.04) (end 77 75) (width 0.25) (layer F.Cu) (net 14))
 (segment (start 77 75) (end 77 61.049) (width 0.25) (layer B.Cu) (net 14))
 (segment (start 77 61.049) (end 72.9507 56.9998) (width 0.25) (layer B.Cu) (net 14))
 (segment (start 72.9507 56.9998) (end 72.1155 56.9998) (width 0.25) (layer F.Cu) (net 14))
 (segment (start 72.1155 56.9998) (end 71.8108 56.695) (width 0.25) (layer F.Cu) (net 14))
 (via (at 77 75) (size 0.6) (layers F.Cu B.Cu) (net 14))
 (via (at 72.9507 56.9998) (size 0.6) (layers F.Cu B.Cu) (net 14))
 (segment (start 62.1892 54.155) (end 61.2242 54.155) (width 0.25) (layer F.Cu) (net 1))
 (segment (start 61.2242 54.155) (end 59.1192 52.05) (width 0.25) (layer F.Cu) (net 1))
 (segment (start 59.1192 52.05) (end 57.1114 52.05) (width 0.25) (layer F.Cu) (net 1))
 (segment (start 57.1114 52.05) (end 53.5 55.6614) (width 0.25) (layer F.Cu) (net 1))
 (segment (start 53.5 55.6614) (end 53.5 59.1532) (width 0.25) (layer F.Cu) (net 1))
 (segment (start 53.5 59.1532) (end 50.4502 62.203) (width 0.25) (layer F.Cu) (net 1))
 (segment (start 50.4502 62.203) (end 50.2 62.203) (width 0.25) (layer F.Cu) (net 1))
 (segment (start 62.1892 56.695) (end 61.2242 56.695) (width 0.25) (layer F.Cu) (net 2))
 (segment (start 61.2242 56.695) (end 57.5292 53) (width 0.25) (layer F.Cu) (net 2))
 (segment (start 57.5292 53) (end 57.4342 53) (width 0.25) (layer F.Cu) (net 2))
 (segment (start 57.4342 53) (end 54.4 56.0342) (width 0.25) (layer F.Cu) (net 2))
 (segment (start 54.4 56.0342) (end 54.4 60.6735) (width 0.25) (layer F.Cu) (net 2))
 (segment (start 54.4 60.6735) (end 51.496 63.5775) (width 0.25) (layer F.Cu) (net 2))
 (segment (start 51.496 63.5775) (end 48.904 63.5775) (width 0.25) (layer F.Cu) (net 2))
 (segment (start 48.904 63.5775) (end 48.5754 63.2489) (width 0.25) (layer F.Cu) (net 2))
 (segment (start 48.5754 63.2489) (end 48.5754 59.5745) (width 0.25) (layer F.Cu) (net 2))
 (segment (start 48.5754 59.5745) (end 49.9498 58.2) (width 0.25) (layer F.Cu) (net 2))
 (segment (start 49.9498 58.2) (end 50.2 58.2) (width 0.25) (layer F.Cu) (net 2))
 (segment (start 50.2 60.2015) (end 49.9498 60.2015) (width 0.25) (layer F.Cu) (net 3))
 (segment (start 49.9498 60.2015) (end 49.0254 61.126) (width 0.25) (layer F.Cu) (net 3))
 (segment (start 49.0254 61.126) (end 49.0254 63.0625) (width 0.25) (layer F.Cu) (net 3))
 (segment (start 49.0254 63.0625) (end 49.0904 63.1275) (width 0.25) (layer F.Cu) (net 3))
 (segment (start 49.0904 63.1275) (end 51.3096 63.1275) (width 0.25) (layer F.Cu) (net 3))
 (segment (start 51.3096 63.1275) (end 53.95 60.4871) (width 0.25) (layer F.Cu) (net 3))
 (segment (start 53.95 60.4871) (end 53.95 55.8478) (width 0.25) (layer F.Cu) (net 3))
 (segment (start 53.95 55.8478) (end 57.2978 52.5) (width 0.25) (layer F.Cu) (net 3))
 (segment (start 57.2978 52.5) (end 58.2992 52.5) (width 0.25) (layer F.Cu) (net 3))
 (segment (start 58.2992 52.5) (end 61.2242 55.425) (width 0.25) (layer F.Cu) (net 3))
 (segment (start 61.2242 55.425) (end 62.1892 55.425) (width 0.25) (layer F.Cu) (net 3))
 (segment (start 62.1892 60.505) (end 62.6287 60.505) (width 0.25) (layer F.Cu) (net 4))
 (segment (start 62.6287 60.505) (end 63.2293 59.9044) (width 0.25) (layer F.Cu) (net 4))
 (segment (start 63.2293 59.9044) (end 63.2293 53.6194) (width 0.25) (layer F.Cu) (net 4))
 (segment (start 63.2293 53.6194) (end 61.1598 51.55) (width 0.25) (layer F.Cu) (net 4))
 (segment (start 61.1598 51.55) (end 56.975 51.55) (width 0.25) (layer F.Cu) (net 4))
 (segment (start 56.975 51.55) (end 52.324 56.201) (width 0.25) (layer F.Cu) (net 4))
 (segment (start 52.324 56.201) (end 50.2 56.201) (width 0.25) (layer F.Cu) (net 4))
 (segment (start 62.1892 63.045) (end 62.6287 63.045) (width 0.25) (layer F.Cu) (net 5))
 (segment (start 62.6287 63.045) (end 63.75 61.9237) (width 0.25) (layer F.Cu) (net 5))
 (segment (start 63.75 61.9237) (end 63.75 60.15) (width 0.25) (layer F.Cu) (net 5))
 (segment (start 63.75 60.15) (end 63.6793 60.0793) (width 0.25) (layer F.Cu) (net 5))
 (segment (start 63.6793 60.0793) (end 63.6793 53.433) (width 0.25) (layer F.Cu) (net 5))
 (segment (start 63.6793 53.433) (end 61.3462 51.1) (width 0.25) (layer F.Cu) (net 5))
 (segment (start 61.3462 51.1) (end 56.725 51.1) (width 0.25) (layer F.Cu) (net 5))
 (segment (start 56.725 51.1) (end 53.6255 54.1995) (width 0.25) (layer F.Cu) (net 5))
 (segment (start 53.6255 54.1995) (end 50.2 54.1995) (width 0.25) (layer F.Cu) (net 5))
 (segment (start 50.5 66) (end 57.6586 66) (width 0.25) (layer F.Cu) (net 8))
 (segment (start 57.6586 66) (end 61.2242 62.4344) (width 0.25) (layer F.Cu) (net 8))
 (segment (start 61.2242 62.4344) (end 61.2242 62.3006) (width 0.25) (layer F.Cu) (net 8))
 (segment (start 61.2242 62.3006) (end 61.7498 61.775) (width 0.25) (layer F.Cu) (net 8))
 (segment (start 61.7498 61.775) (end 62.1892 61.775) (width 0.25) (layer F.Cu) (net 8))
 (segment (start 49.2525 74.5) (end 49.2525 70.8505) (width 0.25) (layer F.Cu) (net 16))
 (segment (start 49.2525 70.8505) (end 49.603 70.5) (width 0.25) (layer F.Cu) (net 16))
 (segment (start 90.197 70.6) (end 93.0525 70.6) (width 0.25) (layer F.Cu) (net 17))
 (segment (start 93.0525 70.6) (end 93.3525 70.3) (width 0.25) (layer F.Cu) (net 17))
 (segment (start 90.297 67.3) (end 92.7525 67.3) (width 0.25) (layer F.Cu) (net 18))
 (segment (start 92.7525 67.3) (end 93.2525 66.8) (width 0.25) (layer F.Cu) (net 18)))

